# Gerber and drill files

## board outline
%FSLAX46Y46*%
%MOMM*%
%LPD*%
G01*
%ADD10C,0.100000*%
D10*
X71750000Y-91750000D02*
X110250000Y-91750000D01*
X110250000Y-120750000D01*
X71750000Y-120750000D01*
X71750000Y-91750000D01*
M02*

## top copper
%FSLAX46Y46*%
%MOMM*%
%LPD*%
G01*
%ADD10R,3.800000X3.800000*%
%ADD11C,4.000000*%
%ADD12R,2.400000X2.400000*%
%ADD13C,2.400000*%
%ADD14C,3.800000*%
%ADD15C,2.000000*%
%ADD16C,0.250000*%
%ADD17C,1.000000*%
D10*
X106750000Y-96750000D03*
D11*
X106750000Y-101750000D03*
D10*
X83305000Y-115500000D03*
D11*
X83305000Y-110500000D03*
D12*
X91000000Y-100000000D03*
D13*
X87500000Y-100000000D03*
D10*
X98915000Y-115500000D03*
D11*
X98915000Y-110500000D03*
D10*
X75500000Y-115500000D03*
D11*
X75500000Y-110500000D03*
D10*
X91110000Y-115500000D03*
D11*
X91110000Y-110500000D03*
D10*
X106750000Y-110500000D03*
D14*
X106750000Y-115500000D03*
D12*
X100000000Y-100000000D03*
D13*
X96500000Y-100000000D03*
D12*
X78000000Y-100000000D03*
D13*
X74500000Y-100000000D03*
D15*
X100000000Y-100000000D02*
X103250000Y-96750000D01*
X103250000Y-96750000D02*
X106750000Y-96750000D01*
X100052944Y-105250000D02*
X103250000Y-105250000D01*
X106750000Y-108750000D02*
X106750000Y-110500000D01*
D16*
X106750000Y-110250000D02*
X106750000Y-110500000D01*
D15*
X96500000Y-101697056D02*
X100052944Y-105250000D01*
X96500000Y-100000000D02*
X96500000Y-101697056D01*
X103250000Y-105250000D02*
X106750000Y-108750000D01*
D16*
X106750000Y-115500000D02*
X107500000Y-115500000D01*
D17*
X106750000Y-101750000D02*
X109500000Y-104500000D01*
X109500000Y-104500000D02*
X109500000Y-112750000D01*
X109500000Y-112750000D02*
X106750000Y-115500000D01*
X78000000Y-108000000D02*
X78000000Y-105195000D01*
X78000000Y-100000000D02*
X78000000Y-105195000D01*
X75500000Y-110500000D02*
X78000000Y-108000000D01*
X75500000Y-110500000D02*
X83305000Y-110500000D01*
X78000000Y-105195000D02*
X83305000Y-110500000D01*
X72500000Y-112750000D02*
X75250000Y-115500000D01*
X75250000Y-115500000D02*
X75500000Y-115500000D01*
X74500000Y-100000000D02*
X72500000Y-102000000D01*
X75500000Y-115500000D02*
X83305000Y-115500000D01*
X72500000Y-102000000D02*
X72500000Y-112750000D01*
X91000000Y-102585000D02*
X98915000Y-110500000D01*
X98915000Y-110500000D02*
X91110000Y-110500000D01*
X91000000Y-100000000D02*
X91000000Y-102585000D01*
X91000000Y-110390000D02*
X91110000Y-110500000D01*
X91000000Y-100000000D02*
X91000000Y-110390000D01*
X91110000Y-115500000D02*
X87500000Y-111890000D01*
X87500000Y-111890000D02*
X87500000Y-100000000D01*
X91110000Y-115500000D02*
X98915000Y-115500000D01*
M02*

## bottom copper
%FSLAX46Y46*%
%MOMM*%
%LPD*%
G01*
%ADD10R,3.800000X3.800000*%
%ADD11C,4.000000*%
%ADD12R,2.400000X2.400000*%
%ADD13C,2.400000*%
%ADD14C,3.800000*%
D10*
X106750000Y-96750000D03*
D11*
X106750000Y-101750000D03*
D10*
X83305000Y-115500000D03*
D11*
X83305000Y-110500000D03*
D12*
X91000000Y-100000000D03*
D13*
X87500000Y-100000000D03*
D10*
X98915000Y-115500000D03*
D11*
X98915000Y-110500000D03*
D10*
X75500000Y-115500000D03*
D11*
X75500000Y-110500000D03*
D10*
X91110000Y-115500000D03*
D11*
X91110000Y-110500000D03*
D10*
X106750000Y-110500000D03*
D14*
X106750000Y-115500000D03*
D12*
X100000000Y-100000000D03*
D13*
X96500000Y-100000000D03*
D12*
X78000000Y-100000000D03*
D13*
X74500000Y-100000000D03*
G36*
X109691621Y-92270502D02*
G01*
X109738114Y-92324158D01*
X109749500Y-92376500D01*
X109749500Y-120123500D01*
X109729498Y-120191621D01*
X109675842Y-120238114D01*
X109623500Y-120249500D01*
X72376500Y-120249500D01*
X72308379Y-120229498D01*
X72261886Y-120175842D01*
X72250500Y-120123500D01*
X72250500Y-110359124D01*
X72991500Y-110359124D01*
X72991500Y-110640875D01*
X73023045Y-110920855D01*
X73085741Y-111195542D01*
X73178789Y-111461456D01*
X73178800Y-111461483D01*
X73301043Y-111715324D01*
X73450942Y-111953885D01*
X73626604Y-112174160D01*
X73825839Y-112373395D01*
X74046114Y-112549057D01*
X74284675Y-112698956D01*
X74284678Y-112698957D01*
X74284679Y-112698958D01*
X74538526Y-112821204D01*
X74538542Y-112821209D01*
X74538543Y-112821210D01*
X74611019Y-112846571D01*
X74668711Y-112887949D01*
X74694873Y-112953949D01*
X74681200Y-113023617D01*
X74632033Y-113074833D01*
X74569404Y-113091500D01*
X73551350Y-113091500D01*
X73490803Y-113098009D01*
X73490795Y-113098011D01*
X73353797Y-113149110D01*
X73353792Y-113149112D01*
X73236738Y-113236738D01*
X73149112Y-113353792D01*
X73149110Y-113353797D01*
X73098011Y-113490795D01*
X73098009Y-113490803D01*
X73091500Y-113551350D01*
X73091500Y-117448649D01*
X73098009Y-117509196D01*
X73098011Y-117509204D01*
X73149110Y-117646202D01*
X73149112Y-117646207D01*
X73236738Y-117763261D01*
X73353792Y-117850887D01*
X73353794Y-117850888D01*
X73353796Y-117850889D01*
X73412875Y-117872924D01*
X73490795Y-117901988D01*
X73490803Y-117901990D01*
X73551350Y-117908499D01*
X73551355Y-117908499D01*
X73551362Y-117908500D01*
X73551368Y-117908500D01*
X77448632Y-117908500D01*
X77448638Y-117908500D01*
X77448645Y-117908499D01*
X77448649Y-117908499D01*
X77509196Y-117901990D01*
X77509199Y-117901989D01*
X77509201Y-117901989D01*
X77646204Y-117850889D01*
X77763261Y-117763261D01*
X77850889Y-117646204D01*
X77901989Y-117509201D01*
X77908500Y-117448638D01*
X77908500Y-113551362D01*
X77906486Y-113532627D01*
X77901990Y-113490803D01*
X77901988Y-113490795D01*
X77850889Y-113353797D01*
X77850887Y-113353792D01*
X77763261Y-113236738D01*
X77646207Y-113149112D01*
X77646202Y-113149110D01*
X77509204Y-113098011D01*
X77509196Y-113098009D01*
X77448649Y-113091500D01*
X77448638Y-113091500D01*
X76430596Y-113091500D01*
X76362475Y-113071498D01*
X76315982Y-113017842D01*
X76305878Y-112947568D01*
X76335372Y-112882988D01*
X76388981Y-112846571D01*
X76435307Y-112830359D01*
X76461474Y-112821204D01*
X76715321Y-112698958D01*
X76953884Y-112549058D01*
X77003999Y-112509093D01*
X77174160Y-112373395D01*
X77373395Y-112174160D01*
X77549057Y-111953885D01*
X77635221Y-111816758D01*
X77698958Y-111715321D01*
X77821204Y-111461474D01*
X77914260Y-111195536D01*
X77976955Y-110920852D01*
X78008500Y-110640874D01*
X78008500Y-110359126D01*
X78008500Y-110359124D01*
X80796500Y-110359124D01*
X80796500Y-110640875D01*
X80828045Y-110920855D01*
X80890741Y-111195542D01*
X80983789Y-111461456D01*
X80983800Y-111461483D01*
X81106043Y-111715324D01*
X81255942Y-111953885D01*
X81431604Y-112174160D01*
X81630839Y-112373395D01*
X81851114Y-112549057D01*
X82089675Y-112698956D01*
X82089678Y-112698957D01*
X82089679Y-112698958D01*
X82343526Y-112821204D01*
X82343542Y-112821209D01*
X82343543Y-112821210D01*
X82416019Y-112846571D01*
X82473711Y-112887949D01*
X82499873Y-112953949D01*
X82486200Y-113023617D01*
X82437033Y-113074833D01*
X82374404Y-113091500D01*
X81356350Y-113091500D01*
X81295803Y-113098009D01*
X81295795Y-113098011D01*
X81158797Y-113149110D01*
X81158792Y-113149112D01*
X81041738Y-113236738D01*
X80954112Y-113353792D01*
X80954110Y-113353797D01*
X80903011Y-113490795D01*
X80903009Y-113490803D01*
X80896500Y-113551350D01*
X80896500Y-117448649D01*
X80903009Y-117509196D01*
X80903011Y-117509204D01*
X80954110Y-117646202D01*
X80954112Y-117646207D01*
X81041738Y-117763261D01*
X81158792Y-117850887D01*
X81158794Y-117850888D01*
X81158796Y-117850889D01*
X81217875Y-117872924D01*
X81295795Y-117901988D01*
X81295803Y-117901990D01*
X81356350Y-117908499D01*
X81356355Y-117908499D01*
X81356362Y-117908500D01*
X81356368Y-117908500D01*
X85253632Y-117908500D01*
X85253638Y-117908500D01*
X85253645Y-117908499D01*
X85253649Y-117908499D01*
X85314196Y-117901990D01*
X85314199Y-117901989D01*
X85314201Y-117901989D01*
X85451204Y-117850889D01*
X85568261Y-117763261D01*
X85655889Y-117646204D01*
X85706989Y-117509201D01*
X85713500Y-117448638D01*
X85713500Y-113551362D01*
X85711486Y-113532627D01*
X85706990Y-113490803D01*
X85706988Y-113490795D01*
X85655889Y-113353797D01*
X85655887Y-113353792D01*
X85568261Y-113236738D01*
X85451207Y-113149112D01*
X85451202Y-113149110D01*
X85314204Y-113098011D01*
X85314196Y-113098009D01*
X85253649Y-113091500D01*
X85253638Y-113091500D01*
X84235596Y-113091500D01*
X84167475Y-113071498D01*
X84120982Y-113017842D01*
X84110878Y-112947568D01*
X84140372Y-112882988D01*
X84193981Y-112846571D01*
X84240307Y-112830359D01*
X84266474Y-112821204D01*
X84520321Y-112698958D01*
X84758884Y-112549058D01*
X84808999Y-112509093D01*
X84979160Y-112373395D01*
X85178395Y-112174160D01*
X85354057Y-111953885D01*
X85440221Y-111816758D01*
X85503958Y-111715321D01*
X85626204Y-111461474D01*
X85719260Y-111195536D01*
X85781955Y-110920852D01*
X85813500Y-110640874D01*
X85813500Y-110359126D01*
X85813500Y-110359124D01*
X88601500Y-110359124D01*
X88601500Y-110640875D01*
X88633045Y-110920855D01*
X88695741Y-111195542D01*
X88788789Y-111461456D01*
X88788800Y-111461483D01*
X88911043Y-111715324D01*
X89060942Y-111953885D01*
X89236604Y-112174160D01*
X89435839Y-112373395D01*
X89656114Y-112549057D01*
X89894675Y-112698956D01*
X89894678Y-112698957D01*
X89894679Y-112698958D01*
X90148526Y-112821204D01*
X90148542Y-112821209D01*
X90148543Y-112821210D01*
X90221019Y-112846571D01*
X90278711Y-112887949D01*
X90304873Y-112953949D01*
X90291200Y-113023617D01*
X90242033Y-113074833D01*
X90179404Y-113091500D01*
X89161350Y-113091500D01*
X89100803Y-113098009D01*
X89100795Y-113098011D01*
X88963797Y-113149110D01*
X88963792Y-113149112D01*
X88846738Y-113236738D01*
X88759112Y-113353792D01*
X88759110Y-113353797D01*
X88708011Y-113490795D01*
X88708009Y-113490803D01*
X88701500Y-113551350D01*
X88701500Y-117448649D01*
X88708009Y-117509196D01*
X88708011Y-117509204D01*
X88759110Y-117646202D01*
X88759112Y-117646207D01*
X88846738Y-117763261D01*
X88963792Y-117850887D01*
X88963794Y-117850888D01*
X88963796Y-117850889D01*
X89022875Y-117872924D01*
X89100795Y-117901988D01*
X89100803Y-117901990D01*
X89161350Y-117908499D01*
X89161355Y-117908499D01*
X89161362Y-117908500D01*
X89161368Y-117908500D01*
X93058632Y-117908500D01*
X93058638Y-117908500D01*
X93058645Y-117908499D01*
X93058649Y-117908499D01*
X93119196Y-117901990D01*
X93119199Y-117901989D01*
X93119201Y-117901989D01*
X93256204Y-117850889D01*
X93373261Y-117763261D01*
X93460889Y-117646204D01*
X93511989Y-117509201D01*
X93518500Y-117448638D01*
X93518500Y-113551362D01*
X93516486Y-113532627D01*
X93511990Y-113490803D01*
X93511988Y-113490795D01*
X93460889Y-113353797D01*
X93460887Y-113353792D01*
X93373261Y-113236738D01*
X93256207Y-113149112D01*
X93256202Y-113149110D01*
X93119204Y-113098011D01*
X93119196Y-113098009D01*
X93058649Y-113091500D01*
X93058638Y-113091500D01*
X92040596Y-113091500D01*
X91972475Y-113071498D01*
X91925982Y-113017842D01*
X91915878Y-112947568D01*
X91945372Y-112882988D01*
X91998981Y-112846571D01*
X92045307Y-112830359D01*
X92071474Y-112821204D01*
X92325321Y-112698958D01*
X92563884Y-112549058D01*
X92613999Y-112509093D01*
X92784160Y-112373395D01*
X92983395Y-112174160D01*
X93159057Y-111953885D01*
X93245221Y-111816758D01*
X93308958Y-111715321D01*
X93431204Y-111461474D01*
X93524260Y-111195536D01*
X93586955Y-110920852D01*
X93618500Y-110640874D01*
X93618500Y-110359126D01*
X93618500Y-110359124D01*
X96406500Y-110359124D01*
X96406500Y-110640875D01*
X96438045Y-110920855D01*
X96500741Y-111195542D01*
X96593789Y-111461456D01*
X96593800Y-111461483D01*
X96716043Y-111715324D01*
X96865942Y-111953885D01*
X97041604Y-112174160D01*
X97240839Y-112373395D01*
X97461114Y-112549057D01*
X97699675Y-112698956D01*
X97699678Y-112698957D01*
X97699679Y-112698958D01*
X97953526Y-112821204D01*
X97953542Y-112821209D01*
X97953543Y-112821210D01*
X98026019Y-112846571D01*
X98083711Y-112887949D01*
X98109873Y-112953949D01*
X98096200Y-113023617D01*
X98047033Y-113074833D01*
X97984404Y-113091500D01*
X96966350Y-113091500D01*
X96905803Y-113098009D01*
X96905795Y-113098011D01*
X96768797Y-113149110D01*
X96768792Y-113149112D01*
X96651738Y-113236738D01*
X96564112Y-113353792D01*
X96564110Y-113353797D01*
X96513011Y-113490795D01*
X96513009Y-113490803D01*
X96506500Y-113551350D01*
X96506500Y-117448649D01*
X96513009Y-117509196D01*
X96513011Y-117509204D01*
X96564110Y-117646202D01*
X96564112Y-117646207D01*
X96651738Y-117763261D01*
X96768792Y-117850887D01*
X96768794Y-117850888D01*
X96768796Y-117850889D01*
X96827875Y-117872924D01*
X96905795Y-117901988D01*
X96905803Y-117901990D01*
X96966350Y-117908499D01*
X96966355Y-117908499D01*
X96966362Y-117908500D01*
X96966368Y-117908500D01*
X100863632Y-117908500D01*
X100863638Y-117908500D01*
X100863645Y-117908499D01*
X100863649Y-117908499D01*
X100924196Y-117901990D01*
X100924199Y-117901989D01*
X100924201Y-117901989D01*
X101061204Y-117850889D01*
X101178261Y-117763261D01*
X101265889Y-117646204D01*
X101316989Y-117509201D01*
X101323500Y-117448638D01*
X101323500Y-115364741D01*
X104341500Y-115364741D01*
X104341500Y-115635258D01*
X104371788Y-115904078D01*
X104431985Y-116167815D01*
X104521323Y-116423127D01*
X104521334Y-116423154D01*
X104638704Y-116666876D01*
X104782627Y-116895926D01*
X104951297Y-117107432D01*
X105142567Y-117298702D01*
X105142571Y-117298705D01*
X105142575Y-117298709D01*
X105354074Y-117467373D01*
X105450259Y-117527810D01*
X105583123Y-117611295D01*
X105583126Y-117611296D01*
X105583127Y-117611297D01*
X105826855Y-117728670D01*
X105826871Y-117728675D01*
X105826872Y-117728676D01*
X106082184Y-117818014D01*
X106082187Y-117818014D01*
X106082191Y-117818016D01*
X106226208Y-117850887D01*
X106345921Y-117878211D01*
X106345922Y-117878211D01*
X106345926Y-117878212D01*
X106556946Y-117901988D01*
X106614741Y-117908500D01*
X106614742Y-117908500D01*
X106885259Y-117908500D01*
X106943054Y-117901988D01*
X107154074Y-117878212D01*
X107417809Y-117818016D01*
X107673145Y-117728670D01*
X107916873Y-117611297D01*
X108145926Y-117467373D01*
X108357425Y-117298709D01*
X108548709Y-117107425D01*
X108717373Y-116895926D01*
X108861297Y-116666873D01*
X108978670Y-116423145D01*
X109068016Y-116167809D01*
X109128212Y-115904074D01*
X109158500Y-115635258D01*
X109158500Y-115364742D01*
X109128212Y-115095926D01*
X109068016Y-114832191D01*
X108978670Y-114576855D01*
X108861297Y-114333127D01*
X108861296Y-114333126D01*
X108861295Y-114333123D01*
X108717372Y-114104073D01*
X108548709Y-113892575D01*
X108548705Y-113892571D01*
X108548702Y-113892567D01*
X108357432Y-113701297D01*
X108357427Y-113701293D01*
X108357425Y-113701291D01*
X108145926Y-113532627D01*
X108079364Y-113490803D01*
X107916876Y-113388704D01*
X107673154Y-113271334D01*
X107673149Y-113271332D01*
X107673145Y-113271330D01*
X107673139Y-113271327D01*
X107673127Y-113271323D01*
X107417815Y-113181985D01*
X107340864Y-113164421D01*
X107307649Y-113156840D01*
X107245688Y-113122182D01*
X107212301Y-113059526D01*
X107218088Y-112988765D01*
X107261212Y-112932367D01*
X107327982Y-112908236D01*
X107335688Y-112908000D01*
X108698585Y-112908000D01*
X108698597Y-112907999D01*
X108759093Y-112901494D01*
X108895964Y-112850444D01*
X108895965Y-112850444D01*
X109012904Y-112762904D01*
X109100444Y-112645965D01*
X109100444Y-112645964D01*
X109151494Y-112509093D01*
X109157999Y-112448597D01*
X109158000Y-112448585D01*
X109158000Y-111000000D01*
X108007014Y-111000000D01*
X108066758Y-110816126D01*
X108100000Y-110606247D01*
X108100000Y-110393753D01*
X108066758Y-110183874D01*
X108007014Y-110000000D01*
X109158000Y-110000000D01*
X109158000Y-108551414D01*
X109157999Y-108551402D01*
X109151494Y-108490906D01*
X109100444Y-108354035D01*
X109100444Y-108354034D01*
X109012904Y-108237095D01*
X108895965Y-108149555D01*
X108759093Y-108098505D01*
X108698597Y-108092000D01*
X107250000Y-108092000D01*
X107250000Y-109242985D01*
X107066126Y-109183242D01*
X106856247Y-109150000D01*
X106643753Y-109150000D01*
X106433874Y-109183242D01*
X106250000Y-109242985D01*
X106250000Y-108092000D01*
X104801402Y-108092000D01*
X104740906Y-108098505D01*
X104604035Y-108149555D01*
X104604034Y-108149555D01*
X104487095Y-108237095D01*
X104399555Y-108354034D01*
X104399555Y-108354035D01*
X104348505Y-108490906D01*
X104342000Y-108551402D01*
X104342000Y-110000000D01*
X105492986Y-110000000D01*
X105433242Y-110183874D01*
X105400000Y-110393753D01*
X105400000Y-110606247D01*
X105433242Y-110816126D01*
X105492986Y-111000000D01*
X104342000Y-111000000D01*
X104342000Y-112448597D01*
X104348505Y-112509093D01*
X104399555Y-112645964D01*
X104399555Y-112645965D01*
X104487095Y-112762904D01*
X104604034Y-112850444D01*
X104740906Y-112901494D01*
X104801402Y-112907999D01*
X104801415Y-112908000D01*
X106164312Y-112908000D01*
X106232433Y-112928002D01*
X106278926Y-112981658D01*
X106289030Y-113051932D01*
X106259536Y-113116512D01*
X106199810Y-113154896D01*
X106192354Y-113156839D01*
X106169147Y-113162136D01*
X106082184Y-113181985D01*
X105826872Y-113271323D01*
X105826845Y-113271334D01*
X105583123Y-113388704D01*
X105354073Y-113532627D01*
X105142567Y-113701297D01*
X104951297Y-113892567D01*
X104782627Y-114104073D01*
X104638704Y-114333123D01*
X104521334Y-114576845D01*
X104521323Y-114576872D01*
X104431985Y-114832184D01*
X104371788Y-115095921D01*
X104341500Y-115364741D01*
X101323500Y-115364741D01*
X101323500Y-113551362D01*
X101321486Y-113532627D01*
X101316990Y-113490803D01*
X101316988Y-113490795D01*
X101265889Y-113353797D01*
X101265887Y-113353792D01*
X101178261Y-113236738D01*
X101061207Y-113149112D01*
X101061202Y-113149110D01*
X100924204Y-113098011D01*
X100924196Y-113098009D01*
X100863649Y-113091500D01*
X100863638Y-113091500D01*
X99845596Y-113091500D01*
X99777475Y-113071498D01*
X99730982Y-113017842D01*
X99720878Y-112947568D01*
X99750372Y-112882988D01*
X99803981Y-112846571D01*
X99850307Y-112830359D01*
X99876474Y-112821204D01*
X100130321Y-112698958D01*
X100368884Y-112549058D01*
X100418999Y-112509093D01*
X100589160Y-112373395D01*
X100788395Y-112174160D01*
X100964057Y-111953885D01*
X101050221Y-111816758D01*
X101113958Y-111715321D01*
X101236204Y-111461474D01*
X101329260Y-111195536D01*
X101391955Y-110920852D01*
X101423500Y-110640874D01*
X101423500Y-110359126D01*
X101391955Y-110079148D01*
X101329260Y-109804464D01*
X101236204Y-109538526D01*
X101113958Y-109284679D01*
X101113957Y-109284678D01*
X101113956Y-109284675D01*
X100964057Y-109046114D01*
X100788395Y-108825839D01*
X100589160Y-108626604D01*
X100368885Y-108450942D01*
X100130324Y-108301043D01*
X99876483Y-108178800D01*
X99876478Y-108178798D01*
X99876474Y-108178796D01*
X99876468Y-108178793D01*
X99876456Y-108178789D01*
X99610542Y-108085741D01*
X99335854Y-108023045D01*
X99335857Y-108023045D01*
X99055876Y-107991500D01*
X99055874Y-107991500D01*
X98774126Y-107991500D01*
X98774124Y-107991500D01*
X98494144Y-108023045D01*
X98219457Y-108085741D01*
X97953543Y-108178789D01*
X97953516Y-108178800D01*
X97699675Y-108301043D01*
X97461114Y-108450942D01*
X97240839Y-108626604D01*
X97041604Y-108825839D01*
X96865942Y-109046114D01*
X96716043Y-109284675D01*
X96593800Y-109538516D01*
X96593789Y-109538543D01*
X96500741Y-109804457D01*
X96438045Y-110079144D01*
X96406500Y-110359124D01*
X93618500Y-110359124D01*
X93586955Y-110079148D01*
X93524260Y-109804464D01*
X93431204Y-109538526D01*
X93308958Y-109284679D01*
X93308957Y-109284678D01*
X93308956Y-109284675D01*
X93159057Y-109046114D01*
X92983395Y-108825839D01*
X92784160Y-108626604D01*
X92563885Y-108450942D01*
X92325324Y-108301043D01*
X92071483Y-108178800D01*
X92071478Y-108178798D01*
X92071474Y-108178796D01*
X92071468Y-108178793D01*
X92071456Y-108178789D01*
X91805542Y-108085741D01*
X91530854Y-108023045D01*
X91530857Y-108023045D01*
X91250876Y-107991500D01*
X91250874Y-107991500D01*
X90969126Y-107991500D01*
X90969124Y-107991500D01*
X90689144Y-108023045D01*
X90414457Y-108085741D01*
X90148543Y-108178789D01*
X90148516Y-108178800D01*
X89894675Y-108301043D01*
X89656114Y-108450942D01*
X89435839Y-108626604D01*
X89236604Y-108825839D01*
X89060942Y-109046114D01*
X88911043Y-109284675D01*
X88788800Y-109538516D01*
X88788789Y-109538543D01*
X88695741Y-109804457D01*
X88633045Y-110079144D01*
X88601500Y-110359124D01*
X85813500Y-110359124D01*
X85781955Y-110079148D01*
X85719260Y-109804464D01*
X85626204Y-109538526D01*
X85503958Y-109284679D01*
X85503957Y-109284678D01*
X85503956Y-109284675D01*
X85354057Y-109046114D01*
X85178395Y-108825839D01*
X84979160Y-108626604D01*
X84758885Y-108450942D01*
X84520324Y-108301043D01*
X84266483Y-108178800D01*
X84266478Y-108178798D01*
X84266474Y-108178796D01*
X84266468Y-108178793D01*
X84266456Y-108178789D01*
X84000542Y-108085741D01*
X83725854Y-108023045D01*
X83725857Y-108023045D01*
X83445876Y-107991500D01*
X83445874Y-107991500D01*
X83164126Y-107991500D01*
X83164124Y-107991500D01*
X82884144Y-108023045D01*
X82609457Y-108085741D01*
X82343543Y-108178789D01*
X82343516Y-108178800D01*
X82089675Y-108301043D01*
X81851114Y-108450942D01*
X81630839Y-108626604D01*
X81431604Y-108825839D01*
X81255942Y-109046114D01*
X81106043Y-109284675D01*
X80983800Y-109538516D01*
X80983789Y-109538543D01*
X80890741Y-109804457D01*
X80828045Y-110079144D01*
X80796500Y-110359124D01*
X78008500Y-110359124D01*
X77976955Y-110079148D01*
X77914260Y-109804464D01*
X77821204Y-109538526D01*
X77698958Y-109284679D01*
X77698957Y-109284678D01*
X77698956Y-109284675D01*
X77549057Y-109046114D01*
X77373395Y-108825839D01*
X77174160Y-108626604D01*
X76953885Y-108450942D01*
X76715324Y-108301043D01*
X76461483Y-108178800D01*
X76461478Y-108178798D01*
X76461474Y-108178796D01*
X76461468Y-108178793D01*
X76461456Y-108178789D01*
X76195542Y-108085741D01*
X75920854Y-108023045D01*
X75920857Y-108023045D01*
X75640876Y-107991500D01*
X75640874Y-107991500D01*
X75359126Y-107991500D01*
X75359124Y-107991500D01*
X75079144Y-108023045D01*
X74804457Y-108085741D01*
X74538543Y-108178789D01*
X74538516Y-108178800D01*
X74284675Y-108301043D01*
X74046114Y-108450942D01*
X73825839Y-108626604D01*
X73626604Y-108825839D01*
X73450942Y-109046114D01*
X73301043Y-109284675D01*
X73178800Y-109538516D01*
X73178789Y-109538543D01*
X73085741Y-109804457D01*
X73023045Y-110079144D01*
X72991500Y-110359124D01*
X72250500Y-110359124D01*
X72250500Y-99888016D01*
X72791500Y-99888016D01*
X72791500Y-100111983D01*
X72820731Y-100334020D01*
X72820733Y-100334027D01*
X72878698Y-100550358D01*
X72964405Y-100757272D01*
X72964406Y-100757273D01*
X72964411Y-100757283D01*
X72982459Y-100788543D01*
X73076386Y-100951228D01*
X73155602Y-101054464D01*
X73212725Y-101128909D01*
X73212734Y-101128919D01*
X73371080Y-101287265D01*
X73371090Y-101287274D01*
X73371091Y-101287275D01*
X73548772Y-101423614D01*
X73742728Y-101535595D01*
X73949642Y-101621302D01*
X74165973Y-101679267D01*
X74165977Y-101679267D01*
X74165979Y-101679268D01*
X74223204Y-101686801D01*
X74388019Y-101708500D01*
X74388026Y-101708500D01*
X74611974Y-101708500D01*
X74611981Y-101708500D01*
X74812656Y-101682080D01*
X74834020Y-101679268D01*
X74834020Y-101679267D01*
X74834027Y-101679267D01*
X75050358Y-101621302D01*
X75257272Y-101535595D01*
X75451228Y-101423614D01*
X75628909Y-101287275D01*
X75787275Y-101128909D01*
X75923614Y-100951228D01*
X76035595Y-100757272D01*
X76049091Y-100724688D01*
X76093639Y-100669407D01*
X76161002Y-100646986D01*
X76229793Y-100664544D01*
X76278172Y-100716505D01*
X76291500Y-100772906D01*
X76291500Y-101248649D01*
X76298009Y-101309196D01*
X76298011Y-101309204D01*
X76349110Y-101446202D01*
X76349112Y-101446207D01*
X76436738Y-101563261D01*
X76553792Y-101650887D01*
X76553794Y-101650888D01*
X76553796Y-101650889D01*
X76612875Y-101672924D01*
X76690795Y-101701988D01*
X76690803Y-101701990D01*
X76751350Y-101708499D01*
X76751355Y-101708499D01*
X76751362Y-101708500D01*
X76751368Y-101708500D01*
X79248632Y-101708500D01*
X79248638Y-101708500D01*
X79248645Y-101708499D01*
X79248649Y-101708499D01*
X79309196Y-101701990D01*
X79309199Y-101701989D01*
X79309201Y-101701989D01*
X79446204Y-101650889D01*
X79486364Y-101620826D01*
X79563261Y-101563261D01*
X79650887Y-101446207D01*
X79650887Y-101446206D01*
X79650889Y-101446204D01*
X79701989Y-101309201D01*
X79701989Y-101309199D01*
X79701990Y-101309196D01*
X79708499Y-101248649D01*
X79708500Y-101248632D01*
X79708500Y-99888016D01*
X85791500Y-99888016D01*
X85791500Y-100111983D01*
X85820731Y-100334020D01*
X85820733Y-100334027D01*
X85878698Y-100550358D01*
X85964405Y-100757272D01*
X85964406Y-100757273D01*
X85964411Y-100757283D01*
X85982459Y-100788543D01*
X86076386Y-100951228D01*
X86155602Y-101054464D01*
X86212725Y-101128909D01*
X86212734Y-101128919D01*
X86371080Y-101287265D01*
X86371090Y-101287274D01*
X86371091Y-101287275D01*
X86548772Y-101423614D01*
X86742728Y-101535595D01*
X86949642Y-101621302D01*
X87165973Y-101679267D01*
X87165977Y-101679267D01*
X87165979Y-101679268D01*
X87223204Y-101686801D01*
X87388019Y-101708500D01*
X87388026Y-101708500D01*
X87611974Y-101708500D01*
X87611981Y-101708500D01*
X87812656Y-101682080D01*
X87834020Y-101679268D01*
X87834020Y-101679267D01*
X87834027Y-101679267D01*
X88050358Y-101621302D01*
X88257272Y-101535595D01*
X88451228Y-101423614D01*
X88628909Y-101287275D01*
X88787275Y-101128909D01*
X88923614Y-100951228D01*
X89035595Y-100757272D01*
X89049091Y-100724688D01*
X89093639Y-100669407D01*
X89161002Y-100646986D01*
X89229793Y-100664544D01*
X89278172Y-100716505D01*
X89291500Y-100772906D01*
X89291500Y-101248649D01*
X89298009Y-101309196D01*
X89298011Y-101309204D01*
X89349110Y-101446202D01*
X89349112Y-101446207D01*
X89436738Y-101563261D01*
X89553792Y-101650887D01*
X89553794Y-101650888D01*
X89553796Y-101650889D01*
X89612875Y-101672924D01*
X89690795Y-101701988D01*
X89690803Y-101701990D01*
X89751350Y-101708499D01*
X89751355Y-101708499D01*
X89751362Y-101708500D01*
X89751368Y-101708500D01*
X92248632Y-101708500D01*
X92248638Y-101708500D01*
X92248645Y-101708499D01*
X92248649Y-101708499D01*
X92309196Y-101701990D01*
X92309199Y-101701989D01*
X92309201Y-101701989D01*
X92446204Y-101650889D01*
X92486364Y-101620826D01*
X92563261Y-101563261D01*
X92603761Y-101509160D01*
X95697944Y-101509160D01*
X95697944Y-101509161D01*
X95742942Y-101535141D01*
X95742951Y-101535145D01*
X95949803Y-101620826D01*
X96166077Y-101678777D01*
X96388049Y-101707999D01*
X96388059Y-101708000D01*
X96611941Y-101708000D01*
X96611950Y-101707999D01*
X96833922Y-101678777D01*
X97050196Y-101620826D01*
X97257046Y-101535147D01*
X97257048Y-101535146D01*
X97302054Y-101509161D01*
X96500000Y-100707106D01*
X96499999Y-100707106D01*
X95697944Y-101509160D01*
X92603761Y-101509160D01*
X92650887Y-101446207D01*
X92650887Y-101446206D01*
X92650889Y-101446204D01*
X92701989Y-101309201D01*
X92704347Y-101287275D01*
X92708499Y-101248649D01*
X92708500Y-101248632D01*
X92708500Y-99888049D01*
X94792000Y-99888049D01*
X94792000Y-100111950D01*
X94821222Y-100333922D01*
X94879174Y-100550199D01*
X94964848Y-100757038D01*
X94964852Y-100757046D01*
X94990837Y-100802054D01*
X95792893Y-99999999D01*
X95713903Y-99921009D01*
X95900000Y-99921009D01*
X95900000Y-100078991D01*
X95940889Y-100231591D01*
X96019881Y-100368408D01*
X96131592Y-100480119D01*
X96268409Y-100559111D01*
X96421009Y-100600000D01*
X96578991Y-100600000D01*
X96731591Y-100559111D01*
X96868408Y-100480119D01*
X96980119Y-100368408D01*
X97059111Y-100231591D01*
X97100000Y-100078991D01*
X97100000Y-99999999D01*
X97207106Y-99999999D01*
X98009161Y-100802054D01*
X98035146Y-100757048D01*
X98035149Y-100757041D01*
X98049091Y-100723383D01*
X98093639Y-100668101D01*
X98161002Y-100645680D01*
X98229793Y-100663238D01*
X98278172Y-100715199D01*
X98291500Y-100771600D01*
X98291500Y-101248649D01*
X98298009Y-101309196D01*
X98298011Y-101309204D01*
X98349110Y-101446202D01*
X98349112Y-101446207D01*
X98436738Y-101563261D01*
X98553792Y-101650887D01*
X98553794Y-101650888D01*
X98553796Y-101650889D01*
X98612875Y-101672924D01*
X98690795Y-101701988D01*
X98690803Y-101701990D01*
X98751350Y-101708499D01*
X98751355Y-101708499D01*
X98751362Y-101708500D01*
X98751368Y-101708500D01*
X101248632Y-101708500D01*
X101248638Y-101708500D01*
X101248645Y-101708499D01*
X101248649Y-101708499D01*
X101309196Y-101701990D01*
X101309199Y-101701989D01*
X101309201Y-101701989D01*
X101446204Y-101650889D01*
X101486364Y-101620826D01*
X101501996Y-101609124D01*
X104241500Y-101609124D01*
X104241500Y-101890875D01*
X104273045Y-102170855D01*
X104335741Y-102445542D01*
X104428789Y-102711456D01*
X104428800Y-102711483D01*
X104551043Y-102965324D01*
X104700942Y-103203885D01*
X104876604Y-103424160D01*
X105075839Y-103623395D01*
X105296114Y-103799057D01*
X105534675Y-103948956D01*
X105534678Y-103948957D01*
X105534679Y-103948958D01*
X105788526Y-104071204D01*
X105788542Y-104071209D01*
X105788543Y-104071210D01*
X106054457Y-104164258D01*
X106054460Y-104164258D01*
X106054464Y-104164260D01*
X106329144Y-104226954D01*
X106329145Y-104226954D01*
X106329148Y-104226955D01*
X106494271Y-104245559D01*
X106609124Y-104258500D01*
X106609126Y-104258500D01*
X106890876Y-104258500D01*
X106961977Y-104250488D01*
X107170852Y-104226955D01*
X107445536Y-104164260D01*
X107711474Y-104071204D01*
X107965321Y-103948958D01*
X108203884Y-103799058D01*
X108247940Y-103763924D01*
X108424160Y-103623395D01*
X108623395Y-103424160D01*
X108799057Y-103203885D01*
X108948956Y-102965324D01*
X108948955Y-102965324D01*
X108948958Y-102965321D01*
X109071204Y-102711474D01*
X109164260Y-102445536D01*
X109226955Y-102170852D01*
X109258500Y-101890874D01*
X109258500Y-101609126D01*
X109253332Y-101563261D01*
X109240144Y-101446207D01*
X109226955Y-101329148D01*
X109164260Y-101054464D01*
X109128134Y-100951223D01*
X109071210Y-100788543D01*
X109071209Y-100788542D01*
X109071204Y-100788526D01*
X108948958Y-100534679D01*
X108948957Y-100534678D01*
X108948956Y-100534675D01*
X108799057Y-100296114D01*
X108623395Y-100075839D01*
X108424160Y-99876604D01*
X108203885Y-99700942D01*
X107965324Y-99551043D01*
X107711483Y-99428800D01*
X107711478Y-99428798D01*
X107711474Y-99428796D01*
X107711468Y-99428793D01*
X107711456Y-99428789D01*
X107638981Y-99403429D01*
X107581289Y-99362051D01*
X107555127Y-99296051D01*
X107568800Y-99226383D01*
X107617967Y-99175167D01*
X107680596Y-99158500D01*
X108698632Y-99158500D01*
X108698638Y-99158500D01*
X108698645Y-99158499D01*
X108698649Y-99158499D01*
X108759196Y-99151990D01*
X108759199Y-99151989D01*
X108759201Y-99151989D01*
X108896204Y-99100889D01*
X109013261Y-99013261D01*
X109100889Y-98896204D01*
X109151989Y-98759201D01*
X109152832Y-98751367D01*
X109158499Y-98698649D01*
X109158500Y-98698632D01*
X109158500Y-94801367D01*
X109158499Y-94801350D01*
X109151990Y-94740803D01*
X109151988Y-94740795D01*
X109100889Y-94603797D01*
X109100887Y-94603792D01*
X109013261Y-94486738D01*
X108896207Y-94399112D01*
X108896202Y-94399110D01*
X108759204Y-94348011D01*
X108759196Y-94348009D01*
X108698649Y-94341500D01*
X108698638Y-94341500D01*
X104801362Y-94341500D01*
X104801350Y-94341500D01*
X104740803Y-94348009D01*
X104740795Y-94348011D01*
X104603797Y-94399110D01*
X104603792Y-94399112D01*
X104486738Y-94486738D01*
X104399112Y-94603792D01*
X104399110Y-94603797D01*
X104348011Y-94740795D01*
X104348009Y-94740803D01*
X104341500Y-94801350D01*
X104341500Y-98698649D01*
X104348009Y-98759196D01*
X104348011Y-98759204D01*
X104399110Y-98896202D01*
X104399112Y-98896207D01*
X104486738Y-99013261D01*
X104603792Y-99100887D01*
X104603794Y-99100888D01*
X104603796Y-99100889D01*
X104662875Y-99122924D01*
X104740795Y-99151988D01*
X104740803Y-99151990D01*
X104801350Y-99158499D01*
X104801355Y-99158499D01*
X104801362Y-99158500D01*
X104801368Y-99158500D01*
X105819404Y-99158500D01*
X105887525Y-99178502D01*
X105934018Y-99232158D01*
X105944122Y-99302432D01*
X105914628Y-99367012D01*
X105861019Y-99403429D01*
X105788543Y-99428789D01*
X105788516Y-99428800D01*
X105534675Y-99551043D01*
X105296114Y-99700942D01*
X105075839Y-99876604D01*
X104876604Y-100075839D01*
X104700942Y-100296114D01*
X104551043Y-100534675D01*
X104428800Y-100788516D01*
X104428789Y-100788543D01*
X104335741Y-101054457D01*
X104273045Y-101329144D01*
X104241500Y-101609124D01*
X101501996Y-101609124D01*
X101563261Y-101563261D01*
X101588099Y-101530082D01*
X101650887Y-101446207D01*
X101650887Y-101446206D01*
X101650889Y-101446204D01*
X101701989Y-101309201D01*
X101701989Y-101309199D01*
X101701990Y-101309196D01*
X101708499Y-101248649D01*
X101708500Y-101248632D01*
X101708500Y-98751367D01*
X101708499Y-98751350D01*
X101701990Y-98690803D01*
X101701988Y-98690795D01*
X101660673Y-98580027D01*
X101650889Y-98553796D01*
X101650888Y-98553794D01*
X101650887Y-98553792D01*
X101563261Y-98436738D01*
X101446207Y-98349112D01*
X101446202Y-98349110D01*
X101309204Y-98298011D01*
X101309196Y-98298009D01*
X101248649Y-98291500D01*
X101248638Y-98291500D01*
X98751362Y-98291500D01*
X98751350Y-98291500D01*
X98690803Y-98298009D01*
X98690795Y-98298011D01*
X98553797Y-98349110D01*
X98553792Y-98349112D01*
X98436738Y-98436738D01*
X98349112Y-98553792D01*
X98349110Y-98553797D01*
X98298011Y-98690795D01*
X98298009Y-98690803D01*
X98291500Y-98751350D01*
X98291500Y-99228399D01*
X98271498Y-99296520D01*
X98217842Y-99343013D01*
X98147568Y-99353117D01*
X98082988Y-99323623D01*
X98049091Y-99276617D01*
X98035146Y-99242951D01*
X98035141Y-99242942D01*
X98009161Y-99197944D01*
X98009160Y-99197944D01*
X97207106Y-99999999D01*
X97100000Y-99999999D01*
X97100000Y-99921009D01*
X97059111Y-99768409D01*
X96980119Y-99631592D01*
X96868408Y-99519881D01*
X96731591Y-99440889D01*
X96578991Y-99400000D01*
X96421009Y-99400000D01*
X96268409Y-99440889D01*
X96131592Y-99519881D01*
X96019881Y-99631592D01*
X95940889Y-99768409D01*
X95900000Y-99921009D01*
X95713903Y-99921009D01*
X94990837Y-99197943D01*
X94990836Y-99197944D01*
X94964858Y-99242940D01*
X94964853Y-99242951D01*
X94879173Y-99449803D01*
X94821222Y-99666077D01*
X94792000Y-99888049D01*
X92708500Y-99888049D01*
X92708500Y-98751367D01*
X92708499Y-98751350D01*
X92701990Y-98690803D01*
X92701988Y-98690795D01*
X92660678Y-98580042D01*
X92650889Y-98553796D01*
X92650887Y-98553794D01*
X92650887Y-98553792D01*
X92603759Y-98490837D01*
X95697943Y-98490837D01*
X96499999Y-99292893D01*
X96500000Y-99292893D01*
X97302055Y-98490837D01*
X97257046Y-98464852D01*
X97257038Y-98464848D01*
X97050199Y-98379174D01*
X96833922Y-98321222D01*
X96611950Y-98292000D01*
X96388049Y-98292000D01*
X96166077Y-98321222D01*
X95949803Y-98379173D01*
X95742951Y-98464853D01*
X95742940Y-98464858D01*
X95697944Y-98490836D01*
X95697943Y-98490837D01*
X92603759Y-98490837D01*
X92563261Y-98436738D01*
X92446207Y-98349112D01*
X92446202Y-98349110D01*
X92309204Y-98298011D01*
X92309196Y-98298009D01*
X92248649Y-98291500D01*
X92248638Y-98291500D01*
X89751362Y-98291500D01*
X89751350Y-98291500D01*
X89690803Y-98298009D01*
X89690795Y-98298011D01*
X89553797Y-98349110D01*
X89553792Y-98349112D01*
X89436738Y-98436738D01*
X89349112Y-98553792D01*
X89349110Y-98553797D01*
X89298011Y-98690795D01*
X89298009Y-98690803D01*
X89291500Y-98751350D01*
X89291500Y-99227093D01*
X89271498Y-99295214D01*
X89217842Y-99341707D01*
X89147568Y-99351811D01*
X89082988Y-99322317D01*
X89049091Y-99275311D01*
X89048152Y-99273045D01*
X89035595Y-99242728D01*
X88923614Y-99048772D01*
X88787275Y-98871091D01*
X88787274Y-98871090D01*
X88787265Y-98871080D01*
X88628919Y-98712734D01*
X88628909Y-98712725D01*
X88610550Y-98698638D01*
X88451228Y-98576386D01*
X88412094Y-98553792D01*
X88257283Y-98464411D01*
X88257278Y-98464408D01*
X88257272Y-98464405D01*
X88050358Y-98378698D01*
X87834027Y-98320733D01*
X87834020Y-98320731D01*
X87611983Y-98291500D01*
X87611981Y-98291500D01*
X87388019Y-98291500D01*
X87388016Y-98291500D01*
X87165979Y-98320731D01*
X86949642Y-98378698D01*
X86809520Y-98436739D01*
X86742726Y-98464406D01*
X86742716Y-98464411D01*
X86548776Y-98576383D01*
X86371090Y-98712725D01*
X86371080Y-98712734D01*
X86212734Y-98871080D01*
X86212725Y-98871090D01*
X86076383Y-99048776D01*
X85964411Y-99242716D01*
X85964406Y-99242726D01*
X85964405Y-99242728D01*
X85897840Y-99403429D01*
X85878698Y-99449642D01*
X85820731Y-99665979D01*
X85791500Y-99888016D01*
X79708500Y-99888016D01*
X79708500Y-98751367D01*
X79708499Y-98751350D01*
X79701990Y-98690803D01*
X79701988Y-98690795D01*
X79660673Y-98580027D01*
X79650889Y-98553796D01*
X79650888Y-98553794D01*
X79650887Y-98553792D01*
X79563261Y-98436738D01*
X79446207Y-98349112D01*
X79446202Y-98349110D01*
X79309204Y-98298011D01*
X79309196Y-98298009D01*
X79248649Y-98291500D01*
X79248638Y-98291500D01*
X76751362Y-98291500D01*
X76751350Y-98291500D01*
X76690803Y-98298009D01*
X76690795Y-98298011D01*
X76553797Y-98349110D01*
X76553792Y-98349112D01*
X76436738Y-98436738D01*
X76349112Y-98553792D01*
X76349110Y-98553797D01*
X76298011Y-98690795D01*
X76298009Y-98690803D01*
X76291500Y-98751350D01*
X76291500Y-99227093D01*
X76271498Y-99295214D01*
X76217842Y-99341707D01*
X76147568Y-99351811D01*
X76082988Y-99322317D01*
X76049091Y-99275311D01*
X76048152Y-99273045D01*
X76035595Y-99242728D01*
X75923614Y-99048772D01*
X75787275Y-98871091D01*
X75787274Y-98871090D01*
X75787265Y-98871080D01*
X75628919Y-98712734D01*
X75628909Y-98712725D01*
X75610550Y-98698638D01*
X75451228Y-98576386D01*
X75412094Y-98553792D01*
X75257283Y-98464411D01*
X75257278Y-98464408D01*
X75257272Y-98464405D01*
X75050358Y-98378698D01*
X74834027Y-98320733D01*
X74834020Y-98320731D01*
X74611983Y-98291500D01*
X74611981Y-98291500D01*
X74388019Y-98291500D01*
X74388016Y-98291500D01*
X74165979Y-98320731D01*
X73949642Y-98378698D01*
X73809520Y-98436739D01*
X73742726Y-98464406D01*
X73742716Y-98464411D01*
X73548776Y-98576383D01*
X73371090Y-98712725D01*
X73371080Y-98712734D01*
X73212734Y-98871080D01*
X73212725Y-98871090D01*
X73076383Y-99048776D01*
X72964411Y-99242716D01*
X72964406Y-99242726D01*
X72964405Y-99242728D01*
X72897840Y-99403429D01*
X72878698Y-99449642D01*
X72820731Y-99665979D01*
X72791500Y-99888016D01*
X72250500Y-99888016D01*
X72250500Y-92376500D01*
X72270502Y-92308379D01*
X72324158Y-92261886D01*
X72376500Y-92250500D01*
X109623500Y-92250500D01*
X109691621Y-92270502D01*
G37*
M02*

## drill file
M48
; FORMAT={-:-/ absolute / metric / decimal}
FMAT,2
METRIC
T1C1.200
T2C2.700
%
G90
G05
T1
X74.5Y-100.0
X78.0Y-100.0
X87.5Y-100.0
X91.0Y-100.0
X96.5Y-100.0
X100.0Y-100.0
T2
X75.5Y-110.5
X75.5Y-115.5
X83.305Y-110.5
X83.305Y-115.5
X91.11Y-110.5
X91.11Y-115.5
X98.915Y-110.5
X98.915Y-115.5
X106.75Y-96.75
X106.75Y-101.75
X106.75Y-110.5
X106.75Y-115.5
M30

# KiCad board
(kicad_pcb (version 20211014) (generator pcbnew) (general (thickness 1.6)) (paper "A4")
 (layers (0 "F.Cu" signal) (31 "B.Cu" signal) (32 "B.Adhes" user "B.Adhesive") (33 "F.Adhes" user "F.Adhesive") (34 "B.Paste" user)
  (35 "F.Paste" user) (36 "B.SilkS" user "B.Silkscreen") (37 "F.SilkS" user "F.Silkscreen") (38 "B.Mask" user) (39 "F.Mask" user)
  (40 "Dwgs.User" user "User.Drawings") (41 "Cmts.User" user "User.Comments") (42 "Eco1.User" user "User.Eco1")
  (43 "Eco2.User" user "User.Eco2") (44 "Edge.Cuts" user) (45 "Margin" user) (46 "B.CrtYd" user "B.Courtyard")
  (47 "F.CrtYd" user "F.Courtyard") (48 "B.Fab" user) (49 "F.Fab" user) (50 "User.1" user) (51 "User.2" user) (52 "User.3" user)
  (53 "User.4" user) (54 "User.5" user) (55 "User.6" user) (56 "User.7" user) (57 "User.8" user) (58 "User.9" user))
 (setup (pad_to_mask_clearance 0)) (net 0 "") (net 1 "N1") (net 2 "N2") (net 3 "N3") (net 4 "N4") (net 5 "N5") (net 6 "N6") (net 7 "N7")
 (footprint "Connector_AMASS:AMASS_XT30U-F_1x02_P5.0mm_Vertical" (layer "F.Cu") (at 106.75 96.75 -90)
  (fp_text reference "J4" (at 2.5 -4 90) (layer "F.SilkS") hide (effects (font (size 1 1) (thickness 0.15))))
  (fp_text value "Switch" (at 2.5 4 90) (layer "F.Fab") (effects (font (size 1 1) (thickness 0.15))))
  (pad "1" thru_hole rect (at 0 0 270) (size 3.8 3.8) (drill 2.7) (layers *.Cu *.Mask) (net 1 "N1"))
  (pad "2" thru_hole circle (at 5 0 270) (size 4 4) (drill 2.7) (layers *.Cu *.Mask) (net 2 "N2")))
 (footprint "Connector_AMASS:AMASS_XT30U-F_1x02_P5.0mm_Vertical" (layer "F.Cu") (at 83.305 115.5 90)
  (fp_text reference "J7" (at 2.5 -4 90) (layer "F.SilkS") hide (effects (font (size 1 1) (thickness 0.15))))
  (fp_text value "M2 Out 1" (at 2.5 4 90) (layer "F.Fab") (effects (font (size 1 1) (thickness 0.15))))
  (pad "1" thru_hole rect (at 0 0 90) (size 3.8 3.8) (drill 2.7) (layers *.Cu *.Mask) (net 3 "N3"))
  (pad "2" thru_hole circle (at 5 0 90) (size 4 4) (drill 2.7) (layers *.Cu *.Mask) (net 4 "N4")))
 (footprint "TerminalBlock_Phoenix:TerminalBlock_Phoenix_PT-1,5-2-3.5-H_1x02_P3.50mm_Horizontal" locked (layer "F.Cu") (at 91 100 180)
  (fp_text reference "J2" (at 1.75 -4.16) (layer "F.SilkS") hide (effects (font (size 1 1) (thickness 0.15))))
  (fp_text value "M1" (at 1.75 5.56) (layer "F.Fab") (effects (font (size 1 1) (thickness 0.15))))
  (pad "1" thru_hole rect locked (at 0 0 180) (size 2.4 2.4) (drill 1.2) (layers *.Cu *.Mask) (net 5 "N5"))
  (pad "2" thru_hole circle locked (at 3.5 0 180) (size 2.4 2.4) (drill 1.2) (layers *.Cu *.Mask) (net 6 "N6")))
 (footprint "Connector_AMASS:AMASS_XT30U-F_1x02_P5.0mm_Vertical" (layer "F.Cu") (at 98.915 115.5 90)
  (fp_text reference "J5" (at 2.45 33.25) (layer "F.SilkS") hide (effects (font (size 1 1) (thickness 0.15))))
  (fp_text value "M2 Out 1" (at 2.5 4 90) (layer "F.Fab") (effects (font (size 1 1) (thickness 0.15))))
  (pad "1" thru_hole rect (at 0 0 90) (size 3.8 3.8) (drill 2.7) (layers *.Cu *.Mask) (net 6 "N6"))
  (pad "2" thru_hole circle (at 5 0 90) (size 4 4) (drill 2.7) (layers *.Cu *.Mask) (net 5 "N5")))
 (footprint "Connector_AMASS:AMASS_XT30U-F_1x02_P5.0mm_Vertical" (layer "F.Cu") (at 75.5 115.5 90)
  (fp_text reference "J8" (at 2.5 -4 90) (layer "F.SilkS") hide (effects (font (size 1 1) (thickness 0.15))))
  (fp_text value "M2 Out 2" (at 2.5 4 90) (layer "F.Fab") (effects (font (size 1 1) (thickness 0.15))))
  (pad "1" thru_hole rect (at 0 0 90) (size 3.8 3.8) (drill 2.7) (layers *.Cu *.Mask) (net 3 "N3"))
  (pad "2" thru_hole circle (at 5 0 90) (size 4 4) (drill 2.7) (layers *.Cu *.Mask) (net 4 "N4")))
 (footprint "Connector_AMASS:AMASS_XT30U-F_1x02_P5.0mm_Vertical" (layer "F.Cu") (at 91.11 115.5 90)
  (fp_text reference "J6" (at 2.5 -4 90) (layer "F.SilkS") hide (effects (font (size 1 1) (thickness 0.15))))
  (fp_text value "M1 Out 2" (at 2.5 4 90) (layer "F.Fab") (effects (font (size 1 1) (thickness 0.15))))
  (pad "1" thru_hole rect (at 0 0 90) (size 3.8 3.8) (drill 2.7) (layers *.Cu *.Mask) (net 6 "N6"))
  (pad "2" thru_hole circle (at 5 0 90) (size 4 4) (drill 2.7) (layers *.Cu *.Mask) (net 5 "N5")))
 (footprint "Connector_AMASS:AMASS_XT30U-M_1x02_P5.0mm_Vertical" (layer "F.Cu") (at 106.75 110.5 -90)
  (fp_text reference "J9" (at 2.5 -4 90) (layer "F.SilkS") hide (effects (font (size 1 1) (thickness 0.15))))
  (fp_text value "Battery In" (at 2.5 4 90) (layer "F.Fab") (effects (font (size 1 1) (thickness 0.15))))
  (pad "1" thru_hole rect (at 0 0 270) (size 3.8 3.8) (drill 2.7) (layers *.Cu *.Mask) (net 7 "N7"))
  (pad "2" thru_hole circle (at 5 0 270) (size 3.8 3.8) (drill 2.7) (layers *.Cu *.Mask) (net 2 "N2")))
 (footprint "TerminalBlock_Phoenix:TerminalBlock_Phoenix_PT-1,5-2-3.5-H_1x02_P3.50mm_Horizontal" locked (layer "F.Cu") (at 100 100 180)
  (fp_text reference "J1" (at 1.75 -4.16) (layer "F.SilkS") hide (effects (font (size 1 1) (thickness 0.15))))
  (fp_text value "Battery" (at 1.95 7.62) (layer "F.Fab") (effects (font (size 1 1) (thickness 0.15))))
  (pad "1" thru_hole rect locked (at 0 0 180) (size 2.4 2.4) (drill 1.2) (layers *.Cu *.Mask) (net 1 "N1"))
  (pad "2" thru_hole circle locked (at 3.5 0 180) (size 2.4 2.4) (drill 1.2) (layers *.Cu *.Mask) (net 7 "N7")))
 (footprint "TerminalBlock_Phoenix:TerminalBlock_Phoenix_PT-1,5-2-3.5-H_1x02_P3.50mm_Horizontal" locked (layer "F.Cu") (at 78 100 180)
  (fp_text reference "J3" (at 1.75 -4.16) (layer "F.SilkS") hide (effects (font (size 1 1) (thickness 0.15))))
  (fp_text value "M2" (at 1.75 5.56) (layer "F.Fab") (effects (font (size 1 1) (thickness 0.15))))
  (pad "1" thru_hole rect locked (at 0 0 180) (size 2.4 2.4) (drill 1.2) (layers *.Cu *.Mask) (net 4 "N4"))
  (pad "2" thru_hole circle locked (at 3.5 0 180) (size 2.4 2.4) (drill 1.2) (layers *.Cu *.Mask) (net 3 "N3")))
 (gr_rect (start 110.25 120.75) (end 71.75 91.75) (layer "Edge.Cuts") (width 0.1) (fill none))
 (segment (start 100 100) (end 103.25 96.75) (width 2) (layer "F.Cu") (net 1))
 (segment (start 103.25 96.75) (end 106.75 96.75) (width 2) (layer "F.Cu") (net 1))
 (segment (start 100.052944 105.25) (end 103.25 105.25) (width 2) (layer "F.Cu") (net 7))
 (segment (start 106.75 108.75) (end 106.75 110.5) (width 2) (layer "F.Cu") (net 7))
 (segment (start 106.75 110.25) (end 106.75 110.5) (width 0.25) (layer "F.Cu") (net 7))
 (segment (start 96.5 101.697056) (end 100.052944 105.25) (width 2) (layer "F.Cu") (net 7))
 (segment (start 96.5 100) (end 96.5 101.697056) (width 2) (layer "F.Cu") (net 7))
 (segment (start 103.25 105.25) (end 106.75 108.75) (width 2) (layer "F.Cu") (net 7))
 (segment (start 106.75 115.5) (end 107.5 115.5) (width 0.25) (layer "F.Cu") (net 2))
 (segment (start 106.75 101.75) (end 109.5 104.5) (width 1) (layer "F.Cu") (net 2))
 (segment (start 109.5 104.5) (end 109.5 112.75) (width 1) (layer "F.Cu") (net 2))
 (segment (start 109.5 112.75) (end 106.75 115.5) (width 1) (layer "F.Cu") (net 2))
 (segment (start 78 108) (end 78 105.195) (width 1) (layer "F.Cu") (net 4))
 (segment (start 78 100) (end 78 105.195) (width 1) (layer "F.Cu") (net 4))
 (segment (start 75.5 110.5) (end 78 108) (width 1) (layer "F.Cu") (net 4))
 (segment (start 75.5 110.5) (end 83.305 110.5) (width 1) (layer "F.Cu") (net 4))
 (segment (start 78 105.195) (end 83.305 110.5) (width 1) (layer "F.Cu") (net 4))
 (segment (start 72.5 112.75) (end 75.25 115.5) (width 1) (layer "F.Cu") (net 3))
 (segment (start 75.25 115.5) (end 75.5 115.5) (width 1) (layer "F.Cu") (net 3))
 (segment (start 74.5 100) (end 72.5 102) (width 1) (layer "F.Cu") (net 3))
 (segment (start 75.5 115.5) (end 83.305 115.5) (width 1) (layer "F.Cu") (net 3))
 (segment (start 72.5 102) (end 72.5 112.75) (width 1) (layer "F.Cu") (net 3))
 (segment (start 91 102.585) (end 98.915 110.5) (width 1) (layer "F.Cu") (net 5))
 (segment (start 98.915 110.5) (end 91.11 110.5) (width 1) (layer "F.Cu") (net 5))
 (segment (start 91 100) (end 91 102.585) (width 1) (layer "F.Cu") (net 5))
 (segment (start 91 110.39) (end 91.11 110.5) (width 1) (layer "F.Cu") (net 5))
 (segment (start 91 100) (end 91 110.39) (width 1) (layer "F.Cu") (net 5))
 (segment (start 91.11 115.5) (end 87.5 111.89) (width 1) (layer "F.Cu") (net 6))
 (segment (start 87.5 111.89) (end 87.5 100) (width 1) (layer "F.Cu") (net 6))
 (segment (start 91.11 115.5) (end 98.915 115.5) (width 1) (layer "F.Cu") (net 6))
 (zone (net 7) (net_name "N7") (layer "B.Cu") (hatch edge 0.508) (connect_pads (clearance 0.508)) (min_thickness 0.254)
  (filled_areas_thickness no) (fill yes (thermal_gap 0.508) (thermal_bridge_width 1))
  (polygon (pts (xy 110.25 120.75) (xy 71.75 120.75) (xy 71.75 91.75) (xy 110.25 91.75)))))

